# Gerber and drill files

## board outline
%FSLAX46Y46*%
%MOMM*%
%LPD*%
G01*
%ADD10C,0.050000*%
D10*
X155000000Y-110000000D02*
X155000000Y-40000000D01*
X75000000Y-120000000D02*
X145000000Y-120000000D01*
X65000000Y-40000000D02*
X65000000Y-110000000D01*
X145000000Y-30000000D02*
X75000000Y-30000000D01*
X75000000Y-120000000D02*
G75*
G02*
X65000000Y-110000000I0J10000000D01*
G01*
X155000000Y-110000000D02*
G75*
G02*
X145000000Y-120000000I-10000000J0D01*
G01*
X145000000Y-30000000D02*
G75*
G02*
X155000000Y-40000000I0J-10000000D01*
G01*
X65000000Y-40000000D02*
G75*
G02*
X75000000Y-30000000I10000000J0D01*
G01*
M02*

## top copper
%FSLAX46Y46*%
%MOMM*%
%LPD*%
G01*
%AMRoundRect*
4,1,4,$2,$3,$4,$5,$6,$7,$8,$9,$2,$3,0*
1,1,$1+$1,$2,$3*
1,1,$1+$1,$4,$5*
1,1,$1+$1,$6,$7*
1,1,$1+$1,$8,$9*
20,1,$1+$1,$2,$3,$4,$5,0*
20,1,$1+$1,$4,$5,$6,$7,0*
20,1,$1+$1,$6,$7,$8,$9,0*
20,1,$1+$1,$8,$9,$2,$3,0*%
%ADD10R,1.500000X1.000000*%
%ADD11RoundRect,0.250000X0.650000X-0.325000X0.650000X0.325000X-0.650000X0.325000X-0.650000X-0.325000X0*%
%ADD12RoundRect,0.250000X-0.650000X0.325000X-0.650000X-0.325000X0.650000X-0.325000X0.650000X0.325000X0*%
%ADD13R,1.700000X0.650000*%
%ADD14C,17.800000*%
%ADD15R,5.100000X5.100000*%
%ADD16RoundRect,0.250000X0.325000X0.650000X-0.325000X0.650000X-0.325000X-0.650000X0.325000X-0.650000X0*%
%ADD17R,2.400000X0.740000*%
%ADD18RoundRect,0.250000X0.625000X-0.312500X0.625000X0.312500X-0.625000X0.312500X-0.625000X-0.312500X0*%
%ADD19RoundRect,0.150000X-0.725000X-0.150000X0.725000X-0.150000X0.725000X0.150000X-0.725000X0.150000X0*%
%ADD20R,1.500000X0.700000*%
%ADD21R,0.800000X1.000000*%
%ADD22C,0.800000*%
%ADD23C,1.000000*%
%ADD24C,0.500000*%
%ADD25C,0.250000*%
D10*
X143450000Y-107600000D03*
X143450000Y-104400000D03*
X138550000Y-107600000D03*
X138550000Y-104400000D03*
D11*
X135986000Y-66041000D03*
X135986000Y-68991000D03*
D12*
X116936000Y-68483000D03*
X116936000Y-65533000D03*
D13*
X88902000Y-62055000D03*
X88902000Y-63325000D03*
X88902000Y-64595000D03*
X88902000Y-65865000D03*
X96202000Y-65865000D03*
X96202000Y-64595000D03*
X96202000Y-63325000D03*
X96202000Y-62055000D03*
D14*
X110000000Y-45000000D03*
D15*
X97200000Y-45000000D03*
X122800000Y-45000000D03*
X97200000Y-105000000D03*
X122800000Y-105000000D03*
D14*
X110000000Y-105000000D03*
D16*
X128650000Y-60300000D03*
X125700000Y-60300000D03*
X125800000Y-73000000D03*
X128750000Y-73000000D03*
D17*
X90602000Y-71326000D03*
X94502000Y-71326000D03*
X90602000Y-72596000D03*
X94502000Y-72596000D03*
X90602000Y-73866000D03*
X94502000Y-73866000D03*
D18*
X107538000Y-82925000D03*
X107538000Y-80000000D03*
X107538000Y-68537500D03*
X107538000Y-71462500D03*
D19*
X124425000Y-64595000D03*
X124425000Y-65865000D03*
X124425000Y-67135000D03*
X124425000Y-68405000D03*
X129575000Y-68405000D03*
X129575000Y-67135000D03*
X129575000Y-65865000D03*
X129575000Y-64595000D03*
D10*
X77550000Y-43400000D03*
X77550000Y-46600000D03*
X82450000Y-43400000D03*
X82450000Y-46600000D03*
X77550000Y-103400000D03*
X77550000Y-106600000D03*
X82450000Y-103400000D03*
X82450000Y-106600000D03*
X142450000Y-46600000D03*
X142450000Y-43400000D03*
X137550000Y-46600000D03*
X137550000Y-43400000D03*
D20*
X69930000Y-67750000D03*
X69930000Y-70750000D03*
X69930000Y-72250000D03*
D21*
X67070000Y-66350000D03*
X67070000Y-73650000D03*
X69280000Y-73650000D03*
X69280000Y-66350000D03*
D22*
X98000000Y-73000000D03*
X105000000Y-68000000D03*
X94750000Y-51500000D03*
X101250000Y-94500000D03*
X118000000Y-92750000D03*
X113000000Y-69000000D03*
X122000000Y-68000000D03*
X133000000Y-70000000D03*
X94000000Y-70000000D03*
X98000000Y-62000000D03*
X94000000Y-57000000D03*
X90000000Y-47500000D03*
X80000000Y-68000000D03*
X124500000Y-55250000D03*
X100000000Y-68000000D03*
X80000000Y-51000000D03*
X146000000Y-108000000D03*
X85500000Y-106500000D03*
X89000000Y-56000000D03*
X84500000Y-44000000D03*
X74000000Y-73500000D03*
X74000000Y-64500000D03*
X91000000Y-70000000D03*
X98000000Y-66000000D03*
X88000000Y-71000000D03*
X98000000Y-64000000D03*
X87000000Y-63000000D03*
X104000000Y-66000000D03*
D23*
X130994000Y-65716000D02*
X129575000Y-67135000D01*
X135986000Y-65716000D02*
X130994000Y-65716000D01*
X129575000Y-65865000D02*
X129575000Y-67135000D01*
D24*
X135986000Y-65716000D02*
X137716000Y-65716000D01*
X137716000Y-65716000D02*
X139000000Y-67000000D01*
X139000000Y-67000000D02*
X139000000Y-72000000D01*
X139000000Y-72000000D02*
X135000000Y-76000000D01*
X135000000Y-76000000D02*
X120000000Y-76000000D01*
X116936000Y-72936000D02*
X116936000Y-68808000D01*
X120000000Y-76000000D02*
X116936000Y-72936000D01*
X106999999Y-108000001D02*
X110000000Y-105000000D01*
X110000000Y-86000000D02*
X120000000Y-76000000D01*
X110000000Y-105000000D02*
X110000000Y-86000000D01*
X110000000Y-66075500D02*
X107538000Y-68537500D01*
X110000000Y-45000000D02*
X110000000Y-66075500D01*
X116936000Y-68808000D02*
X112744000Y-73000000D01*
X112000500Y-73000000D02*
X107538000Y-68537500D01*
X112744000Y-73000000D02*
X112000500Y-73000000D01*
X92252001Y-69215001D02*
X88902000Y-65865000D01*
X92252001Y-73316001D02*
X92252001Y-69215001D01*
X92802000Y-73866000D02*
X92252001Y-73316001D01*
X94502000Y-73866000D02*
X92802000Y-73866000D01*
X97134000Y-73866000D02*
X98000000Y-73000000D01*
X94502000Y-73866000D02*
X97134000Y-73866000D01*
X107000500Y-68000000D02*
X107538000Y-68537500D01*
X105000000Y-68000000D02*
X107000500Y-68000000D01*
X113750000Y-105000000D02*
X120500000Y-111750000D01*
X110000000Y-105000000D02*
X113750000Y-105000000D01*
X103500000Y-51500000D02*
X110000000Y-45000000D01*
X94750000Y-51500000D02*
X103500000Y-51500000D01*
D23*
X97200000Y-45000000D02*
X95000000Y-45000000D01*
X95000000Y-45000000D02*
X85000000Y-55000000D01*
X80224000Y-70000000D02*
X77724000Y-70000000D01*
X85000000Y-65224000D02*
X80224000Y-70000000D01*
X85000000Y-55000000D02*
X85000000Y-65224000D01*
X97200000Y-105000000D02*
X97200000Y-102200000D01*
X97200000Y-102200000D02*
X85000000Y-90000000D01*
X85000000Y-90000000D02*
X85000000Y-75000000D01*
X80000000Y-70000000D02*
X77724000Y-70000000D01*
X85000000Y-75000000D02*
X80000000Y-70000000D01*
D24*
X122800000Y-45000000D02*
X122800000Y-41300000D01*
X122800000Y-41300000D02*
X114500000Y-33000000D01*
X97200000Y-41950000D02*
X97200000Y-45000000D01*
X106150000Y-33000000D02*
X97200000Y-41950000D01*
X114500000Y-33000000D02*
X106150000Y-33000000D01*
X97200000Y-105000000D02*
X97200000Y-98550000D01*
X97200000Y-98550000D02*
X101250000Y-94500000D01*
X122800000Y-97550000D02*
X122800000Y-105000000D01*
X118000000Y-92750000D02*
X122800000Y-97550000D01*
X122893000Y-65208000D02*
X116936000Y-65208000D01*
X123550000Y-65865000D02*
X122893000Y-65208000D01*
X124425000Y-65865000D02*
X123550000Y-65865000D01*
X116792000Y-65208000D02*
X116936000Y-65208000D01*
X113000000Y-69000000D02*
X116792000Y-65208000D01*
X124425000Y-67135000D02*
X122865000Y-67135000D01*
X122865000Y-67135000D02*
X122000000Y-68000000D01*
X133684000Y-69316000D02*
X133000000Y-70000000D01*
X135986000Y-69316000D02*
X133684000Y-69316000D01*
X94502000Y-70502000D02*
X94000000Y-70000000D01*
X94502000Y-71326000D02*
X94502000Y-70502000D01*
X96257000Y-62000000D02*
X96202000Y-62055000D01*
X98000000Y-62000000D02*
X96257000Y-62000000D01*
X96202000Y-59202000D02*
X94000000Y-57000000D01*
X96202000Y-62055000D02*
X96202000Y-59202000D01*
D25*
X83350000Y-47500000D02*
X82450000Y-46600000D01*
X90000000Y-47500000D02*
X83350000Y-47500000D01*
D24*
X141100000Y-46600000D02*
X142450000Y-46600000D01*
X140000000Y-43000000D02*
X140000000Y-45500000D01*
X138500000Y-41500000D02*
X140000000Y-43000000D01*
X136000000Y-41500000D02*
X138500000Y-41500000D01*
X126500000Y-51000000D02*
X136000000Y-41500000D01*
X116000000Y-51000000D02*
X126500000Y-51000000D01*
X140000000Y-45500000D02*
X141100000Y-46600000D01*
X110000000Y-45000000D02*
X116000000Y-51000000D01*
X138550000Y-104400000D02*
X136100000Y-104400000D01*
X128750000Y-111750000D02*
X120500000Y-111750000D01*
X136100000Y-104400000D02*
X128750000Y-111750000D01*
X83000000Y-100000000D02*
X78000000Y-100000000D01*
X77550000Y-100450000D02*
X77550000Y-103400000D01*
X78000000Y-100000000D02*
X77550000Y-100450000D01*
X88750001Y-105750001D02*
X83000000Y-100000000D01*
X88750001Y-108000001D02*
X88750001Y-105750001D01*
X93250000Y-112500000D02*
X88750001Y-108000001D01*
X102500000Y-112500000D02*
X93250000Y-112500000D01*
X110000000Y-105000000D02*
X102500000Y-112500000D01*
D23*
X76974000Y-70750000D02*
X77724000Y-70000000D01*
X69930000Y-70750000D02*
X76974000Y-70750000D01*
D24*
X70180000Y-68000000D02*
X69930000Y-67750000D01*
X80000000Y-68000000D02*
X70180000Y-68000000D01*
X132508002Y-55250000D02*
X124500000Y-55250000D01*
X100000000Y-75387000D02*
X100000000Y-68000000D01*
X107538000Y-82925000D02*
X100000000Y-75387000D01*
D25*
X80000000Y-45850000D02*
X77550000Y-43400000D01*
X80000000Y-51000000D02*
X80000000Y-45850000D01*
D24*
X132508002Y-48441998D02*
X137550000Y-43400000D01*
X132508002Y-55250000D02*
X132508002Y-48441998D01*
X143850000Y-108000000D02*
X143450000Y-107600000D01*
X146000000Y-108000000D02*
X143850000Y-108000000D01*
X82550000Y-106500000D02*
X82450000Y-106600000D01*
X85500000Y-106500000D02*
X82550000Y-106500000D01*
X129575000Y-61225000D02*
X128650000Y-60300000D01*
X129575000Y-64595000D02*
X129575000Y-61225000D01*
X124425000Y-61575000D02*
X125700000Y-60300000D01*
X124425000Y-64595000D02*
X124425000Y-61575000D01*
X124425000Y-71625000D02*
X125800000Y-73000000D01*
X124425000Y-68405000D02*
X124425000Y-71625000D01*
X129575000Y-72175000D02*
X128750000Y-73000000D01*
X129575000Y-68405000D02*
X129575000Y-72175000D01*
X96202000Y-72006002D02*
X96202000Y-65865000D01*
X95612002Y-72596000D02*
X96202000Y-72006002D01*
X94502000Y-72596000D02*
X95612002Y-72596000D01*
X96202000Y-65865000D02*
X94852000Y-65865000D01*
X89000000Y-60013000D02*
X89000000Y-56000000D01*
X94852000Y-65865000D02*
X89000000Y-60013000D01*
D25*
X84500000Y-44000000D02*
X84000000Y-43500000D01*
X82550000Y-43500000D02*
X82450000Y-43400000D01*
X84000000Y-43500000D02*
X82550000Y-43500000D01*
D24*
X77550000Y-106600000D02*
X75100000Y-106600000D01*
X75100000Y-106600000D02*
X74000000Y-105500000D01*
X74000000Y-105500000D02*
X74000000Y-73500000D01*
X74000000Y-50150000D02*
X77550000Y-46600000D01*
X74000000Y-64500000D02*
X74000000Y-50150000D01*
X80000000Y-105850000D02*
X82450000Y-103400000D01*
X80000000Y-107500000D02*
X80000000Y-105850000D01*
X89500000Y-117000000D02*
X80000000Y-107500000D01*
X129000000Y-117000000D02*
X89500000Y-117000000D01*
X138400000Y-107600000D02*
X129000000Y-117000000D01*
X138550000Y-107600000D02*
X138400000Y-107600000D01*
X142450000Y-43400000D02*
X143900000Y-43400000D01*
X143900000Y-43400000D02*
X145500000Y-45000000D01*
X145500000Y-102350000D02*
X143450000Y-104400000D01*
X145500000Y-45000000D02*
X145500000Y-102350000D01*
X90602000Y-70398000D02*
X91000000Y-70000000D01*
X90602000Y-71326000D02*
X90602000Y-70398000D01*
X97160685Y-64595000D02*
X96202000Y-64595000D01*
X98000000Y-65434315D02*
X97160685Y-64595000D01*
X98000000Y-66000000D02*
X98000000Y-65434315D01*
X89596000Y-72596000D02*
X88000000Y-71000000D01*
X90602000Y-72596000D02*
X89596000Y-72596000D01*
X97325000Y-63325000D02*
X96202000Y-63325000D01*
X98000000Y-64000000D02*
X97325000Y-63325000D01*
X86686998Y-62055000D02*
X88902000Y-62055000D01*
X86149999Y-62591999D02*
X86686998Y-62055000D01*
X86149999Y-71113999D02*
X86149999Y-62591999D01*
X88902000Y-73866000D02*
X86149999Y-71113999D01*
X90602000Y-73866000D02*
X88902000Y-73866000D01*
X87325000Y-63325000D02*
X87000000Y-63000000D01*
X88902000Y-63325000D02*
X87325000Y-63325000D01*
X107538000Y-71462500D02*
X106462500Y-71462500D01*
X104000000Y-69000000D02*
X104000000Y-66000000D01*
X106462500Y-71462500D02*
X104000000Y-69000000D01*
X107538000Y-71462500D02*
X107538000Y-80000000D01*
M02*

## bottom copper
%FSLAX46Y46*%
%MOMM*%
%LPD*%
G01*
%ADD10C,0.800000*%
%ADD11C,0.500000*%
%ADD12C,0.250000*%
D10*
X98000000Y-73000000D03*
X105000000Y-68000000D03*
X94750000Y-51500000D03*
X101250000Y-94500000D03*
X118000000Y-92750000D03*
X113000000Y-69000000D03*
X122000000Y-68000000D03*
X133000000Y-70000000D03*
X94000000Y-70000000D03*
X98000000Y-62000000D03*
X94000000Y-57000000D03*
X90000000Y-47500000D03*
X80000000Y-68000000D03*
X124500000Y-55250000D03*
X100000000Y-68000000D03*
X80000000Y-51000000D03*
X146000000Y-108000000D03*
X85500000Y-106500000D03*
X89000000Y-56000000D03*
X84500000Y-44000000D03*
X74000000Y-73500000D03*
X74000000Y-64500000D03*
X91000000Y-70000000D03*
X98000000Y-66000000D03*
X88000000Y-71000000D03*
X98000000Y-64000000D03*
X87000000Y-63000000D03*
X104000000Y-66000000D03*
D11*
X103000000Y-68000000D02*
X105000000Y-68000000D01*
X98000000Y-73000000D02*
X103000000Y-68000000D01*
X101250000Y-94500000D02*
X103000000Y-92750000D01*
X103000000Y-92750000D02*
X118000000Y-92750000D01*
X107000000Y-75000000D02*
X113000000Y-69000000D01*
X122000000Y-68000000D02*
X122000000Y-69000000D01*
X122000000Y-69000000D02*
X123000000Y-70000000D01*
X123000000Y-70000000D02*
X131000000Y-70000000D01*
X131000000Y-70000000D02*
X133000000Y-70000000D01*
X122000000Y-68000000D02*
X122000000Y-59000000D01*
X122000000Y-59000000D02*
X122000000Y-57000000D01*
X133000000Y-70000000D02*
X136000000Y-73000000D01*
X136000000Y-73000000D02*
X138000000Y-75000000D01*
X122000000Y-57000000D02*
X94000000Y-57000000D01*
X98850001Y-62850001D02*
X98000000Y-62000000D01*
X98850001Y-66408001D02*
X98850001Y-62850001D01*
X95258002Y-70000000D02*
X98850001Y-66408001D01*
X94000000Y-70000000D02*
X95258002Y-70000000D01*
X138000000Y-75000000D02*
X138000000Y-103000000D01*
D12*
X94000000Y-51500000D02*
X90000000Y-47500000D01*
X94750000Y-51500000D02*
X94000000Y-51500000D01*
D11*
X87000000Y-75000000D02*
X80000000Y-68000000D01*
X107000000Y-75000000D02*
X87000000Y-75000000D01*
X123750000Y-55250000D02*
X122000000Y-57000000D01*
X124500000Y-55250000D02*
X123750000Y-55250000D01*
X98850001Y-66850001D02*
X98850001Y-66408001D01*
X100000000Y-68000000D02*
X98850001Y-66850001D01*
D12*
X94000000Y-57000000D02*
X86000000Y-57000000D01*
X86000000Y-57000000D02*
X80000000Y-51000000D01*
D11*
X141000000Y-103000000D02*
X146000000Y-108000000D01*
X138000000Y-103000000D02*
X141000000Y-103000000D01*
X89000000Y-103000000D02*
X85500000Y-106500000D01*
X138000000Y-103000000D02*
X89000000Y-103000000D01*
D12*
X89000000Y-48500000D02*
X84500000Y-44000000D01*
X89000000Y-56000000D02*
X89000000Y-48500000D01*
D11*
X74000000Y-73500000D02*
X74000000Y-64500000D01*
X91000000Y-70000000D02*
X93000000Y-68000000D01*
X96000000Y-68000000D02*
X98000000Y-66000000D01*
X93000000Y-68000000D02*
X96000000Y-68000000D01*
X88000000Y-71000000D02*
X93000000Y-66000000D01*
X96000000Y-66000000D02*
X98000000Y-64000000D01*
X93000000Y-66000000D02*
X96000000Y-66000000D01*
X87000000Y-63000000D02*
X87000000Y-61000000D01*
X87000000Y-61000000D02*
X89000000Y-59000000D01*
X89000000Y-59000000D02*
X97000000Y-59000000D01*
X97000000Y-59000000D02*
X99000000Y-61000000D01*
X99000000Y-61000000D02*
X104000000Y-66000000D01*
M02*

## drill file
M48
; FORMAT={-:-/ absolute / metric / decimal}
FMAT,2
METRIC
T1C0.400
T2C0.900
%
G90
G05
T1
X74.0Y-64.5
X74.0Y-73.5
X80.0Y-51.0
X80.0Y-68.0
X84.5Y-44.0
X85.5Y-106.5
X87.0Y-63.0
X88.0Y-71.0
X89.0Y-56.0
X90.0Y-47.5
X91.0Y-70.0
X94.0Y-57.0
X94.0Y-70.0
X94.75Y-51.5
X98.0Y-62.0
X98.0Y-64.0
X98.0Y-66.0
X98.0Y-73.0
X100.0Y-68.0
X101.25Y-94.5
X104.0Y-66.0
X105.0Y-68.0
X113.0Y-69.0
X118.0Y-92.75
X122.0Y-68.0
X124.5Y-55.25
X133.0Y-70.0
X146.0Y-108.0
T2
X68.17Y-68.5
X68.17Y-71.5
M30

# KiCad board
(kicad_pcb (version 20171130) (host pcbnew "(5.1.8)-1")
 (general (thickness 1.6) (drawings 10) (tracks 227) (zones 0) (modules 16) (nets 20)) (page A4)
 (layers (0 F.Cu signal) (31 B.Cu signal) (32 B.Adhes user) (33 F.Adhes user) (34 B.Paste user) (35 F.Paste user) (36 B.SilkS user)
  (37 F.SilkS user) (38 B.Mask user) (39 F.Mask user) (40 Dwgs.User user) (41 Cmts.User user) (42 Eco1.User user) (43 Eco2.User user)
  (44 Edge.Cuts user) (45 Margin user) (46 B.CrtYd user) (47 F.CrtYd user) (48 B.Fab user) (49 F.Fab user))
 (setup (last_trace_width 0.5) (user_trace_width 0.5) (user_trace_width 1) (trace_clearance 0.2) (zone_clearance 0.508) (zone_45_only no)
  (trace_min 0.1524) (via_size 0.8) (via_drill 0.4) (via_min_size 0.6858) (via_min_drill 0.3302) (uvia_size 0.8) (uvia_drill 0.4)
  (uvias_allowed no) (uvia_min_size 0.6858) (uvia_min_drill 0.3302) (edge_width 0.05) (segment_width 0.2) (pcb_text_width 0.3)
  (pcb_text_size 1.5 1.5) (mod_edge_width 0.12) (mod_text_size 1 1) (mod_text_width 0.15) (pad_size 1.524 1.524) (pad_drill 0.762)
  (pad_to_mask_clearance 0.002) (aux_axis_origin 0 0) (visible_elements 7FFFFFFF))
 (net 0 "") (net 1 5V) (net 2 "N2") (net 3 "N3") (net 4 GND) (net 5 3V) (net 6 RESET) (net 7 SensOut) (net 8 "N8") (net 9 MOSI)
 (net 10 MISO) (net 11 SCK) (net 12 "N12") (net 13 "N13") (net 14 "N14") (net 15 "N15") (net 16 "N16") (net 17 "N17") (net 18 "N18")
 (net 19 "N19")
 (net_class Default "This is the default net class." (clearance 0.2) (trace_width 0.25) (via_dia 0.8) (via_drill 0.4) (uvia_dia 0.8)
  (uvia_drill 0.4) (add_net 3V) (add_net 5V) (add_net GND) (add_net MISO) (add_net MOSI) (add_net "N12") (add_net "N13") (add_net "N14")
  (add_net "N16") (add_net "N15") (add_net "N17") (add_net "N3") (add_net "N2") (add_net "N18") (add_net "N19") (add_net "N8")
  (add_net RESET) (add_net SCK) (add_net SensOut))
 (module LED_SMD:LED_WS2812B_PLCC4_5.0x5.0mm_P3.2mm (layer F.Cu) (at 141 106 180)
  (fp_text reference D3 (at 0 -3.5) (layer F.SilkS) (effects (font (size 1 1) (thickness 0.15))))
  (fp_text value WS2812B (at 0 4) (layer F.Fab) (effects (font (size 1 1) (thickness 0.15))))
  (pad 1 smd rect (at -2.45 -1.6 180) (size 1.5 1) (layers F.Cu F.Paste F.Mask) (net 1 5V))
  (pad 2 smd rect (at -2.45 1.6 180) (size 1.5 1) (layers F.Cu F.Paste F.Mask) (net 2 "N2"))
  (pad 4 smd rect (at 2.45 -1.6 180) (size 1.5 1) (layers F.Cu F.Paste F.Mask) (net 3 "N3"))
  (pad 3 smd rect (at 2.45 1.6 180) (size 1.5 1) (layers F.Cu F.Paste F.Mask) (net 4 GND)))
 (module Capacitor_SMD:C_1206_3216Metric (layer F.Cu) (at 135.986 67.516 90)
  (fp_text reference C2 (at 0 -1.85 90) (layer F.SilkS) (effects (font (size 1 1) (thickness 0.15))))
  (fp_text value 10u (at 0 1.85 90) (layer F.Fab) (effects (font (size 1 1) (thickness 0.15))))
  (pad 2 smd roundrect (at 1.475 0 90) (size 1.15 1.8) (layers F.Cu F.Paste F.Mask) (roundrect_rratio 0.217391) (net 4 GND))
  (pad 1 smd roundrect (at -1.475 0 90) (size 1.15 1.8) (layers F.Cu F.Paste F.Mask) (roundrect_rratio 0.217391) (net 1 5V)))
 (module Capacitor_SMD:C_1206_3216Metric (layer F.Cu) (at 116.936 67.008 270)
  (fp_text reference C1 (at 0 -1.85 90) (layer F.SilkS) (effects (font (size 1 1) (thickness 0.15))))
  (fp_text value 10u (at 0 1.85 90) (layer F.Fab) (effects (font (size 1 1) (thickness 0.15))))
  (pad 2 smd roundrect (at 1.475 0 270) (size 1.15 1.8) (layers F.Cu F.Paste F.Mask) (roundrect_rratio 0.217391) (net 4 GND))
  (pad 1 smd roundrect (at -1.475 0 270) (size 1.15 1.8) (layers F.Cu F.Paste F.Mask) (roundrect_rratio 0.217391) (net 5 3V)))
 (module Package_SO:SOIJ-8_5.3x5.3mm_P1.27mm (layer F.Cu) (at 92.552 63.96)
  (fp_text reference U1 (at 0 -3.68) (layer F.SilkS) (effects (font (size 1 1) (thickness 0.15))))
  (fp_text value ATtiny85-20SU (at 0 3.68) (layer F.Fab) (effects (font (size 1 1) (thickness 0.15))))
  (pad 1 smd rect (at -3.65 -1.905) (size 1.7 0.65) (layers F.Cu F.Paste F.Mask) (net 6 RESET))
  (pad 2 smd rect (at -3.65 -0.635) (size 1.7 0.65) (layers F.Cu F.Paste F.Mask) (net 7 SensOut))
  (pad 3 smd rect (at -3.65 0.635) (size 1.7 0.65) (layers F.Cu F.Paste F.Mask) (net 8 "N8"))
  (pad 4 smd rect (at -3.65 1.905) (size 1.7 0.65) (layers F.Cu F.Paste F.Mask) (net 4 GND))
  (pad 5 smd rect (at 3.65 1.905) (size 1.7 0.65) (layers F.Cu F.Paste F.Mask) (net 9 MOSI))
  (pad 6 smd rect (at 3.65 0.635) (size 1.7 0.65) (layers F.Cu F.Paste F.Mask) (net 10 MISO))
  (pad 7 smd rect (at 3.65 -0.635) (size 1.7 0.65) (layers F.Cu F.Paste F.Mask) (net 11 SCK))
  (pad 8 smd rect (at 3.65 -1.905) (size 1.7 0.65) (layers F.Cu F.Paste F.Mask) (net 1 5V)))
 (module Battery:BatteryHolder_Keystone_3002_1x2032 (layer F.Cu) (at 110 45)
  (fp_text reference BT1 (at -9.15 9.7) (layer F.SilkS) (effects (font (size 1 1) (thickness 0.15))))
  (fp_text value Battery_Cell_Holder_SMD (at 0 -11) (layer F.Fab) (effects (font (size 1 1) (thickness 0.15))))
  (pad 2 smd circle (at 0 0) (size 17.8 17.8) (layers F.Cu F.Mask) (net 4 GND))
  (pad 1 smd rect (at -12.8 0) (size 5.1 5.1) (layers F.Cu F.Paste F.Mask) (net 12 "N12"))
  (pad 1 smd rect (at 12.8 0) (size 5.1 5.1) (layers F.Cu F.Paste F.Mask) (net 12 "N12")))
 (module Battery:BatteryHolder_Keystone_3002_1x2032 (layer F.Cu) (at 110 105 180)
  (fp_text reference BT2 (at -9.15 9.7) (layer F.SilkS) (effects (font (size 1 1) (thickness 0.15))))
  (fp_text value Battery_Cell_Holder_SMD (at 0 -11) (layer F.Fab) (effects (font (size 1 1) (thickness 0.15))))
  (pad 1 smd rect (at 12.8 0 180) (size 5.1 5.1) (layers F.Cu F.Paste F.Mask) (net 12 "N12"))
  (pad 1 smd rect (at -12.8 0 180) (size 5.1 5.1) (layers F.Cu F.Paste F.Mask) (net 12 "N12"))
  (pad 2 smd circle (at 0 0 180) (size 17.8 17.8) (layers F.Cu F.Mask) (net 4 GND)))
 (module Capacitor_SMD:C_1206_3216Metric (layer F.Cu) (at 127.175 60.3 180)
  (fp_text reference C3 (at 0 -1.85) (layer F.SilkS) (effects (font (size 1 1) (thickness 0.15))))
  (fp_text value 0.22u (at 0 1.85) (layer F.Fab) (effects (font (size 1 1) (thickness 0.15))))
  (pad 1 smd roundrect (at -1.475 0 180) (size 1.15 1.8) (layers F.Cu F.Paste F.Mask) (roundrect_rratio 0.217391) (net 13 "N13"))
  (pad 2 smd roundrect (at 1.475 0 180) (size 1.15 1.8) (layers F.Cu F.Paste F.Mask) (roundrect_rratio 0.217391) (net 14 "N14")))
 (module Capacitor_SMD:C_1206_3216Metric (layer F.Cu) (at 127.275 73 180)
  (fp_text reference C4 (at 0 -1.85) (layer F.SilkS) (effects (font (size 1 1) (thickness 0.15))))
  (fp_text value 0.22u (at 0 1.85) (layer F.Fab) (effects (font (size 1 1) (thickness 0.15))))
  (pad 2 smd roundrect (at 1.475 0 180) (size 1.15 1.8) (layers F.Cu F.Paste F.Mask) (roundrect_rratio 0.217391) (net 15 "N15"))
  (pad 1 smd roundrect (at -1.475 0 180) (size 1.15 1.8) (layers F.Cu F.Paste F.Mask) (roundrect_rratio 0.217391) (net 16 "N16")))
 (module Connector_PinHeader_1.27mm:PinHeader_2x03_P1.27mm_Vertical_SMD (layer F.Cu) (at 92.552 72.596)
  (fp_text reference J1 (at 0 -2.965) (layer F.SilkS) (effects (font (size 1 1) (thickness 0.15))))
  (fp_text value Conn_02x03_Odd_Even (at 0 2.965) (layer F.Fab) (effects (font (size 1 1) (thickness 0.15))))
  (pad 1 smd rect (at -1.95 -1.27) (size 2.4 0.74) (layers F.Cu F.Paste F.Mask) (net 10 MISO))
  (pad 2 smd rect (at 1.95 -1.27) (size 2.4 0.74) (layers F.Cu F.Paste F.Mask) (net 1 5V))
  (pad 3 smd rect (at -1.95 0) (size 2.4 0.74) (layers F.Cu F.Paste F.Mask) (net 11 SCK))
  (pad 4 smd rect (at 1.95 0) (size 2.4 0.74) (layers F.Cu F.Paste F.Mask) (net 9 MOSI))
  (pad 5 smd rect (at -1.95 1.27) (size 2.4 0.74) (layers F.Cu F.Paste F.Mask) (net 6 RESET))
  (pad 6 smd rect (at 1.95 1.27) (size 2.4 0.74) (layers F.Cu F.Paste F.Mask) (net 4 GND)))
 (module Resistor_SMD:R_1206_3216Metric (layer F.Cu) (at 107.538 81.4625 90)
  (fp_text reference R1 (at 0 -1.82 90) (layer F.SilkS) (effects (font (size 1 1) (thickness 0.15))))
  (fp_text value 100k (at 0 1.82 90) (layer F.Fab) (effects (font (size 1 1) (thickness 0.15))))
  (pad 1 smd roundrect (at -1.4625 0 90) (size 1.125 1.75) (layers F.Cu F.Paste F.Mask) (roundrect_rratio 0.222222) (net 1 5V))
  (pad 2 smd roundrect (at 1.4625 0 90) (size 1.125 1.75) (layers F.Cu F.Paste F.Mask) (roundrect_rratio 0.222222) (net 7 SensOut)))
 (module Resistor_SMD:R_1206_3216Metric (layer F.Cu) (at 107.538 70 90)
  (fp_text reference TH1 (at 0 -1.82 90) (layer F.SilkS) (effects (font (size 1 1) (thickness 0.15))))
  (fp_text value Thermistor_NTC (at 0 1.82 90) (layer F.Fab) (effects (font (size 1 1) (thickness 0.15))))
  (pad 2 smd roundrect (at 1.4625 0 90) (size 1.125 1.75) (layers F.Cu F.Paste F.Mask) (roundrect_rratio 0.222222) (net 4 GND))
  (pad 1 smd roundrect (at -1.4625 0 90) (size 1.125 1.75) (layers F.Cu F.Paste F.Mask) (roundrect_rratio 0.222222) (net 7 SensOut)))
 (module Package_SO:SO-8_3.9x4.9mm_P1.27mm (layer F.Cu) (at 127 66.5)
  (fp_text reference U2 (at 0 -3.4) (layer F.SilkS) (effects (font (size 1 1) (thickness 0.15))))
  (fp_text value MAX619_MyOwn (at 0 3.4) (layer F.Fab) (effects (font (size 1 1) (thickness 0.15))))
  (pad 1 smd roundrect (at -2.575 -1.905) (size 1.75 0.6) (layers F.Cu F.Paste F.Mask) (roundrect_rratio 0.25) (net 14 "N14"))
  (pad 2 smd roundrect (at -2.575 -0.635) (size 1.75 0.6) (layers F.Cu F.Paste F.Mask) (roundrect_rratio 0.25) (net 5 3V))
  (pad 3 smd roundrect (at -2.575 0.635) (size 1.75 0.6) (layers F.Cu F.Paste F.Mask) (roundrect_rratio 0.25) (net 1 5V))
  (pad 4 smd roundrect (at -2.575 1.905) (size 1.75 0.6) (layers F.Cu F.Paste F.Mask) (roundrect_rratio 0.25) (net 15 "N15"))
  (pad 5 smd roundrect (at 2.575 1.905) (size 1.75 0.6) (layers F.Cu F.Paste F.Mask) (roundrect_rratio 0.25) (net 16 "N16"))
  (pad 6 smd roundrect (at 2.575 0.635) (size 1.75 0.6) (layers F.Cu F.Paste F.Mask) (roundrect_rratio 0.25) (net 4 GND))
  (pad 7 smd roundrect (at 2.575 -0.635) (size 1.75 0.6) (layers F.Cu F.Paste F.Mask) (roundrect_rratio 0.25) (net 4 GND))
  (pad 8 smd roundrect (at 2.575 -1.905) (size 1.75 0.6) (layers F.Cu F.Paste F.Mask) (roundrect_rratio 0.25) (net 13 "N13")))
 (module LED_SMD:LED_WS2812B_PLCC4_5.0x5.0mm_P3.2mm (layer F.Cu) (at 80 45)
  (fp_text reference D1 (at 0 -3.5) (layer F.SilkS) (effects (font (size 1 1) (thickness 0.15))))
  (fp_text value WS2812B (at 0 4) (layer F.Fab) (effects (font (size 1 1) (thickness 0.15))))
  (pad 1 smd rect (at -2.45 -1.6) (size 1.5 1) (layers F.Cu F.Paste F.Mask) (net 1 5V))
  (pad 2 smd rect (at -2.45 1.6) (size 1.5 1) (layers F.Cu F.Paste F.Mask) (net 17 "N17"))
  (pad 4 smd rect (at 2.45 -1.6) (size 1.5 1) (layers F.Cu F.Paste F.Mask) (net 9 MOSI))
  (pad 3 smd rect (at 2.45 1.6) (size 1.5 1) (layers F.Cu F.Paste F.Mask) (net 4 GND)))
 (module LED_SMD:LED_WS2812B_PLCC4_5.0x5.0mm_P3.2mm (layer F.Cu) (at 80 105 180)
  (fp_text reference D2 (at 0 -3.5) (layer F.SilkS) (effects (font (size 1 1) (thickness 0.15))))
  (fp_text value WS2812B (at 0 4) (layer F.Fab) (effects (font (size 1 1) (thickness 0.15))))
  (pad 3 smd rect (at 2.45 1.6 180) (size 1.5 1) (layers F.Cu F.Paste F.Mask) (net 4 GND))
  (pad 4 smd rect (at 2.45 -1.6 180) (size 1.5 1) (layers F.Cu F.Paste F.Mask) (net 17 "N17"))
  (pad 2 smd rect (at -2.45 1.6 180) (size 1.5 1) (layers F.Cu F.Paste F.Mask) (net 3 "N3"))
  (pad 1 smd rect (at -2.45 -1.6 180) (size 1.5 1) (layers F.Cu F.Paste F.Mask) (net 1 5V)))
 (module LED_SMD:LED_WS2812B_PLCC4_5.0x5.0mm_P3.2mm (layer F.Cu) (at 140 45)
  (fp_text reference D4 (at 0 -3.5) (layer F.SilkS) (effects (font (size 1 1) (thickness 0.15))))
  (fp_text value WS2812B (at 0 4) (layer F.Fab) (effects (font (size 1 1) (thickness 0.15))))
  (pad 3 smd rect (at 2.45 1.6) (size 1.5 1) (layers F.Cu F.Paste F.Mask) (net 4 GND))
  (pad 4 smd rect (at 2.45 -1.6) (size 1.5 1) (layers F.Cu F.Paste F.Mask) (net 2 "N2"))
  (pad 2 smd rect (at -2.45 1.6) (size 1.5 1) (layers F.Cu F.Paste F.Mask) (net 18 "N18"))
  (pad 1 smd rect (at -2.45 -1.6) (size 1.5 1) (layers F.Cu F.Paste F.Mask) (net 1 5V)))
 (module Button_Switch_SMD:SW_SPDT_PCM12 (layer F.Cu) (at 68.5 70 270)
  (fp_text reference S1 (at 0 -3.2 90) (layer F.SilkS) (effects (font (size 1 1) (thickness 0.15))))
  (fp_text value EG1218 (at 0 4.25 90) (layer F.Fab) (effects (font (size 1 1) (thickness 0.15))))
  (pad "" np_thru_hole circle (at -1.5 0.33 270) (size 0.9 0.9) (drill 0.9) (layers *.Cu *.Mask))
  (pad "" np_thru_hole circle (at 1.5 0.33 270) (size 0.9 0.9) (drill 0.9) (layers *.Cu *.Mask))
  (pad 1 smd rect (at -2.25 -1.43 270) (size 0.7 1.5) (layers F.Cu F.Paste F.Mask) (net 5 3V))
  (pad 2 smd rect (at 0.75 -1.43 270) (size 0.7 1.5) (layers F.Cu F.Paste F.Mask) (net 12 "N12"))
  (pad 3 smd rect (at 2.25 -1.43 270) (size 0.7 1.5) (layers F.Cu F.Paste F.Mask) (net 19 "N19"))
  (pad "" smd rect (at -3.65 1.43 270) (size 1 0.8) (layers F.Cu F.Paste F.Mask))
  (pad "" smd rect (at 3.65 1.43 270) (size 1 0.8) (layers F.Cu F.Paste F.Mask))
  (pad "" smd rect (at 3.65 -0.78 270) (size 1 0.8) (layers F.Cu F.Paste F.Mask))
  (pad "" smd rect (at -3.65 -0.78 270) (size 1 0.8) (layers F.Cu F.Paste F.Mask)))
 (gr_line (start 155 110) (end 155 40) (layer Edge.Cuts) (width 0.05))
 (gr_line (start 75 120) (end 145 120) (layer Edge.Cuts) (width 0.05))
 (gr_line (start 65 40) (end 65 110) (layer Edge.Cuts) (width 0.05))
 (gr_line (start 145 30) (end 75 30) (layer Edge.Cuts) (width 0.05))
 (gr_arc (start 75 110) (end 65 110) (angle -90) (layer Edge.Cuts) (width 0.05))
 (gr_arc (start 145 110) (end 145 120) (angle -90) (layer Edge.Cuts) (width 0.05))
 (gr_arc (start 145 40) (end 155 40) (angle -90) (layer Edge.Cuts) (width 0.05))
 (gr_arc (start 75 40) (end 75 30) (angle -90) (layer Edge.Cuts) (width 0.05))
 (segment (start 130.994 65.716) (end 129.575 67.135) (width 1) (layer F.Cu) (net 4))
 (segment (start 135.986 65.716) (end 130.994 65.716) (width 1) (layer F.Cu) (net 4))
 (segment (start 129.575 65.865) (end 129.575 67.135) (width 1) (layer F.Cu) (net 4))
 (segment (start 135.986 65.716) (end 137.716 65.716) (width 0.5) (layer F.Cu) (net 4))
 (segment (start 137.716 65.716) (end 139 67) (width 0.5) (layer F.Cu) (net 4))
 (segment (start 139 67) (end 139 72) (width 0.5) (layer F.Cu) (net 4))
 (segment (start 139 72) (end 135 76) (width 0.5) (layer F.Cu) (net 4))
 (segment (start 135 76) (end 120 76) (width 0.5) (layer F.Cu) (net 4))
 (segment (start 116.936 72.936) (end 116.936 68.808) (width 0.5) (layer F.Cu) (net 4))
 (segment (start 120 76) (end 116.936 72.936) (width 0.5) (layer F.Cu) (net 4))
 (segment (start 106.999999 108.000001) (end 110 105) (width 0.5) (layer F.Cu) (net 4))
 (segment (start 110 86) (end 120 76) (width 0.5) (layer F.Cu) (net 4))
 (segment (start 110 105) (end 110 86) (width 0.5) (layer F.Cu) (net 4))
 (segment (start 110 66.0755) (end 107.538 68.5375) (width 0.5) (layer F.Cu) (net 4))
 (segment (start 110 45) (end 110 66.0755) (width 0.5) (layer F.Cu) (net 4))
 (segment (start 116.936 68.808) (end 112.744 73) (width 0.5) (layer F.Cu) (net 4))
 (segment (start 112.0005 73) (end 107.538 68.5375) (width 0.5) (layer F.Cu) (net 4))
 (segment (start 112.744 73) (end 112.0005 73) (width 0.5) (layer F.Cu) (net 4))
 (segment (start 92.252001 69.215001) (end 88.902 65.865) (width 0.5) (layer F.Cu) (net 4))
 (segment (start 92.252001 73.316001) (end 92.252001 69.215001) (width 0.5) (layer F.Cu) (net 4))
 (segment (start 92.802 73.866) (end 92.252001 73.316001) (width 0.5) (layer F.Cu) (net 4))
 (segment (start 94.502 73.866) (end 92.802 73.866) (width 0.5) (layer F.Cu) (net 4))
 (via (at 98 73) (size 0.8) (drill 0.4) (layers F.Cu B.Cu) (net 4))
 (segment (start 97.134 73.866) (end 98 73) (width 0.5) (layer F.Cu) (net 4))
 (segment (start 94.502 73.866) (end 97.134 73.866) (width 0.5) (layer F.Cu) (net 4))
 (via (at 105 68) (size 0.8) (drill 0.4) (layers F.Cu B.Cu) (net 4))
 (segment (start 103 68) (end 105 68) (width 0.5) (layer B.Cu) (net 4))
 (segment (start 98 73) (end 103 68) (width 0.5) (layer B.Cu) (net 4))
 (segment (start 107.0005 68) (end 107.538 68.5375) (width 0.5) (layer F.Cu) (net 4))
 (segment (start 105 68) (end 107.0005 68) (width 0.5) (layer F.Cu) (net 4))
 (segment (start 113.75 105) (end 120.5 111.75) (width 0.5) (layer F.Cu) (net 4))
 (segment (start 110 105) (end 113.75 105) (width 0.5) (layer F.Cu) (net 4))
 (via (at 94.75 51.5) (size 0.8) (drill 0.4) (layers F.Cu B.Cu) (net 4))
 (segment (start 103.5 51.5) (end 110 45) (width 0.5) (layer F.Cu) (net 4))
 (segment (start 94.75 51.5) (end 103.5 51.5) (width 0.5) (layer F.Cu) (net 4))
 (segment (start 97.2 45) (end 95 45) (width 1) (layer F.Cu) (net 12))
 (segment (start 95 45) (end 85 55) (width 1) (layer F.Cu) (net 12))
 (segment (start 80.224 70) (end 77.724 70) (width 1) (layer F.Cu) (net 12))
 (segment (start 85 65.224) (end 80.224 70) (width 1) (layer F.Cu) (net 12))
 (segment (start 85 55) (end 85 65.224) (width 1) (layer F.Cu) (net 12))
 (segment (start 97.2 105) (end 97.2 102.2) (width 1) (layer F.Cu) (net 12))
 (segment (start 97.2 102.2) (end 85 90) (width 1) (layer F.Cu) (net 12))
 (segment (start 85 90) (end 85 75) (width 1) (layer F.Cu) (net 12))
 (segment (start 80 70) (end 77.724 70) (width 1) (layer F.Cu) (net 12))
 (segment (start 85 75) (end 80 70) (width 1) (layer F.Cu) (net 12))
 (segment (start 122.8 45) (end 122.8 41.3) (width 0.5) (layer F.Cu) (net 12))
 (segment (start 122.8 41.3) (end 114.5 33) (width 0.5) (layer F.Cu) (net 12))
 (segment (start 97.2 41.95) (end 97.2 45) (width 0.5) (layer F.Cu) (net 12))
 (segment (start 106.15 33) (end 97.2 41.95) (width 0.5) (layer F.Cu) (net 12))
 (segment (start 114.5 33) (end 106.15 33) (width 0.5) (layer F.Cu) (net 12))
 (segment (start 97.2 105) (end 97.2 98.55) (width 0.5) (layer F.Cu) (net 12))
 (via (at 101.25 94.5) (size 0.8) (drill 0.4) (layers F.Cu B.Cu) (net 12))
 (segment (start 97.2 98.55) (end 101.25 94.5) (width 0.5) (layer F.Cu) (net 12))
 (segment (start 101.25 94.5) (end 103 92.75) (width 0.5) (layer B.Cu) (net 12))
 (via (at 118 92.75) (size 0.8) (drill 0.4) (layers F.Cu B.Cu) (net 12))
 (segment (start 103 92.75) (end 118 92.75) (width 0.5) (layer B.Cu) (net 12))
 (segment (start 122.8 97.55) (end 122.8 105) (width 0.5) (layer F.Cu) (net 12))
 (segment (start 118 92.75) (end 122.8 97.55) (width 0.5) (layer F.Cu) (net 12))
 (segment (start 122.893 65.208) (end 116.936 65.208) (width 0.5) (layer F.Cu) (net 5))
 (segment (start 123.55 65.865) (end 122.893 65.208) (width 0.5) (layer F.Cu) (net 5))
 (segment (start 124.425 65.865) (end 123.55 65.865) (width 0.5) (layer F.Cu) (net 5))
 (via (at 113 69) (size 0.8) (drill 0.4) (layers F.Cu B.Cu) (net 5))
 (segment (start 107 75) (end 113 69) (width 0.5) (layer B.Cu) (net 5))
 (segment (start 116.792 65.208) (end 116.936 65.208) (width 0.5) (layer F.Cu) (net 5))
 (segment (start 113 69) (end 116.792 65.208) (width 0.5) (layer F.Cu) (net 5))
 (segment (start 124.425 67.135) (end 122.865 67.135) (width 0.5) (layer F.Cu) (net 1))
 (via (at 122 68) (size 0.8) (drill 0.4) (layers F.Cu B.Cu) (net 1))
 (segment (start 122.865 67.135) (end 122 68) (width 0.5) (layer F.Cu) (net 1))
 (segment (start 122 68) (end 122 69) (width 0.5) (layer B.Cu) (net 1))
 (segment (start 122 69) (end 123 70) (width 0.5) (layer B.Cu) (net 1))
 (segment (start 123 70) (end 131 70) (width 0.5) (layer B.Cu) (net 1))
 (segment (start 131 70) (end 133 70) (width 0.5) (layer B.Cu) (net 1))
 (via (at 133 70) (size 0.8) (drill 0.4) (layers F.Cu B.Cu) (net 1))
 (segment (start 133.684 69.316) (end 133 70) (width 0.5) (layer F.Cu) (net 1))
 (segment (start 135.986 69.316) (end 133.684 69.316) (width 0.5) (layer F.Cu) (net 1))
 (segment (start 122 68) (end 122 59) (width 0.5) (layer B.Cu) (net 1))
 (segment (start 122 59) (end 122 57) (width 0.5) (layer B.Cu) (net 1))
 (segment (start 133 70) (end 136 73) (width 0.5) (layer B.Cu) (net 1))
 (segment (start 136 73) (end 138 75) (width 0.5) (layer B.Cu) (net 1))
 (segment (start 122 57) (end 94 57) (width 0.5) (layer B.Cu) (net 1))
 (via (at 94 70) (size 0.8) (drill 0.4) (layers F.Cu B.Cu) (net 1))
 (segment (start 94.502 70.502) (end 94 70) (width 0.5) (layer F.Cu) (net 1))
 (segment (start 94.502 71.326) (end 94.502 70.502) (width 0.5) (layer F.Cu) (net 1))
 (via (at 98 62) (size 0.8) (drill 0.4) (layers F.Cu B.Cu) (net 1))
 (segment (start 98.850001 62.850001) (end 98 62) (width 0.5) (layer B.Cu) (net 1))
 (segment (start 98.850001 66.408001) (end 98.850001 62.850001) (width 0.5) (layer B.Cu) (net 1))
 (segment (start 95.258002 70) (end 98.850001 66.408001) (width 0.5) (layer B.Cu) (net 1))
 (segment (start 94 70) (end 95.258002 70) (width 0.5) (layer B.Cu) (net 1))
 (segment (start 96.257 62) (end 96.202 62.055) (width 0.5) (layer F.Cu) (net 1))
 (segment (start 98 62) (end 96.257 62) (width 0.5) (layer F.Cu) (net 1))
 (via (at 94 57) (size 0.8) (drill 0.4) (layers F.Cu B.Cu) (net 1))
 (segment (start 96.202 59.202) (end 94 57) (width 0.5) (layer F.Cu) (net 1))
 (segment (start 96.202 62.055) (end 96.202 59.202) (width 0.5) (layer F.Cu) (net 1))
 (segment (start 138 75) (end 138 103) (width 0.5) (layer B.Cu) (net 1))
 (via (at 90 47.5) (size 0.8) (drill 0.4) (layers F.Cu B.Cu) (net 4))
 (segment (start 94 51.5) (end 90 47.5) (width 0.25) (layer B.Cu) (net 4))
 (segment (start 94.75 51.5) (end 94 51.5) (width 0.25) (layer B.Cu) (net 4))
 (segment (start 83.35 47.5) (end 82.45 46.6) (width 0.25) (layer F.Cu) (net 4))
 (segment (start 90 47.5) (end 83.35 47.5) (width 0.25) (layer F.Cu) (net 4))
 (segment (start 141.1 46.6) (end 142.45 46.6) (width 0.5) (layer F.Cu) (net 4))
 (segment (start 140 43) (end 140 45.5) (width 0.5) (layer F.Cu) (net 4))
 (segment (start 138.5 41.5) (end 140 43) (width 0.5) (layer F.Cu) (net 4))
 (segment (start 136 41.5) (end 138.5 41.5) (width 0.5) (layer F.Cu) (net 4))
 (segment (start 126.5 51) (end 136 41.5) (width 0.5) (layer F.Cu) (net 4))
 (segment (start 116 51) (end 126.5 51) (width 0.5) (layer F.Cu) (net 4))
 (segment (start 140 45.5) (end 141.1 46.6) (width 0.5) (layer F.Cu) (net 4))
 (segment (start 110 45) (end 116 51) (width 0.5) (layer F.Cu) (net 4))
 (segment (start 138.55 104.4) (end 136.1 104.4) (width 0.5) (layer F.Cu) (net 4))
 (segment (start 128.75 111.75) (end 120.5 111.75) (width 0.5) (layer F.Cu) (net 4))
 (segment (start 136.1 104.4) (end 128.75 111.75) (width 0.5) (layer F.Cu) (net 4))
 (segment (start 83 100) (end 78 100) (width 0.5) (layer F.Cu) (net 4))
 (segment (start 77.55 100.45) (end 77.55 103.4) (width 0.5) (layer F.Cu) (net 4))
 (segment (start 78 100) (end 77.55 100.45) (width 0.5) (layer F.Cu) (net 4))
 (segment (start 88.750001 105.750001) (end 83 100) (width 0.5) (layer F.Cu) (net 4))
 (segment (start 88.750001 108.000001) (end 88.750001 105.750001) (width 0.5) (layer F.Cu) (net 4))
 (segment (start 93.25 112.5) (end 88.750001 108.000001) (width 0.5) (layer F.Cu) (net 4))
 (segment (start 102.5 112.5) (end 93.25 112.5) (width 0.5) (layer F.Cu) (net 4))
 (segment (start 110 105) (end 102.5 112.5) (width 0.5) (layer F.Cu) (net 4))
 (segment (start 76.974 70.75) (end 77.724 70) (width 1) (layer F.Cu) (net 12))
 (segment (start 69.93 70.75) (end 76.974 70.75) (width 1) (layer F.Cu) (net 12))
 (via (at 80 68) (size 0.8) (drill 0.4) (layers F.Cu B.Cu) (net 5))
 (segment (start 87 75) (end 80 68) (width 0.5) (layer B.Cu) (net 5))
 (segment (start 107 75) (end 87 75) (width 0.5) (layer B.Cu) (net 5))
 (segment (start 70.18 68) (end 69.93 67.75) (width 0.5) (layer F.Cu) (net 5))
 (segment (start 80 68) (end 70.18 68) (width 0.5) (layer F.Cu) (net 5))
 (via (at 124.5 55.25) (size 0.8) (drill 0.4) (layers F.Cu B.Cu) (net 1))
 (segment (start 132.508002 55.25) (end 124.5 55.25) (width 0.5) (layer F.Cu) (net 1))
 (segment (start 123.75 55.25) (end 122 57) (width 0.5) (layer B.Cu) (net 1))
 (segment (start 124.5 55.25) (end 123.75 55.25) (width 0.5) (layer B.Cu) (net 1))
 (via (at 100 68) (size 0.8) (drill 0.4) (layers F.Cu B.Cu) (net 1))
 (segment (start 100 75.387) (end 100 68) (width 0.5) (layer F.Cu) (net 1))
 (segment (start 107.538 82.925) (end 100 75.387) (width 0.5) (layer F.Cu) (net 1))
 (segment (start 98.850001 66.850001) (end 98.850001 66.408001) (width 0.5) (layer B.Cu) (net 1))
 (segment (start 100 68) (end 98.850001 66.850001) (width 0.5) (layer B.Cu) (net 1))
 (segment (start 94 57) (end 86 57) (width 0.25) (layer B.Cu) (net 1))
 (via (at 80 51) (size 0.8) (drill 0.4) (layers F.Cu B.Cu) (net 1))
 (segment (start 86 57) (end 80 51) (width 0.25) (layer B.Cu) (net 1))
 (segment (start 80 45.85) (end 77.55 43.4) (width 0.25) (layer F.Cu) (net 1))
 (segment (start 80 51) (end 80 45.85) (width 0.25) (layer F.Cu) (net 1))
 (segment (start 132.508002 48.441998) (end 137.55 43.4) (width 0.5) (layer F.Cu) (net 1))
 (segment (start 132.508002 55.25) (end 132.508002 48.441998) (width 0.5) (layer F.Cu) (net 1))
 (via (at 146 108) (size 0.8) (drill 0.4) (layers F.Cu B.Cu) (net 1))
 (segment (start 141 103) (end 146 108) (width 0.5) (layer B.Cu) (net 1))
 (segment (start 138 103) (end 141 103) (width 0.5) (layer B.Cu) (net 1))
 (segment (start 143.85 108) (end 143.45 107.6) (width 0.5) (layer F.Cu) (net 1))
 (segment (start 146 108) (end 143.85 108) (width 0.5) (layer F.Cu) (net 1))
 (via (at 85.5 106.5) (size 0.8) (drill 0.4) (layers F.Cu B.Cu) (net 1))
 (segment (start 89 103) (end 85.5 106.5) (width 0.5) (layer B.Cu) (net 1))
 (segment (start 138 103) (end 89 103) (width 0.5) (layer B.Cu) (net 1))
 (segment (start 82.55 106.5) (end 82.45 106.6) (width 0.5) (layer F.Cu) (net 1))
 (segment (start 85.5 106.5) (end 82.55 106.5) (width 0.5) (layer F.Cu) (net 1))
 (segment (start 129.575 61.225) (end 128.65 60.3) (width 0.5) (layer F.Cu) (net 13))
 (segment (start 129.575 64.595) (end 129.575 61.225) (width 0.5) (layer F.Cu) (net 13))
 (segment (start 124.425 61.575) (end 125.7 60.3) (width 0.5) (layer F.Cu) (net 14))
 (segment (start 124.425 64.595) (end 124.425 61.575) (width 0.5) (layer F.Cu) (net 14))
 (segment (start 124.425 71.625) (end 125.8 73) (width 0.5) (layer F.Cu) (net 15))
 (segment (start 124.425 68.405) (end 124.425 71.625) (width 0.5) (layer F.Cu) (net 15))
 (segment (start 129.575 72.175) (end 128.75 73) (width 0.5) (layer F.Cu) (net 16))
 (segment (start 129.575 68.405) (end 129.575 72.175) (width 0.5) (layer F.Cu) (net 16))
 (segment (start 96.202 72.006002) (end 96.202 65.865) (width 0.5) (layer F.Cu) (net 9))
 (segment (start 95.612002 72.596) (end 96.202 72.006002) (width 0.5) (layer F.Cu) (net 9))
 (segment (start 94.502 72.596) (end 95.612002 72.596) (width 0.5) (layer F.Cu) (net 9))
 (via (at 89 56) (size 0.8) (drill 0.4) (layers F.Cu B.Cu) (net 9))
 (segment (start 96.202 65.865) (end 94.852 65.865) (width 0.5) (layer F.Cu) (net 9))
 (segment (start 89 60.013) (end 89 56) (width 0.5) (layer F.Cu) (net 9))
 (segment (start 94.852 65.865) (end 89 60.013) (width 0.5) (layer F.Cu) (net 9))
 (via (at 84.5 44) (size 0.8) (drill 0.4) (layers F.Cu B.Cu) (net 9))
 (segment (start 89 48.5) (end 84.5 44) (width 0.25) (layer B.Cu) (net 9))
 (segment (start 89 56) (end 89 48.5) (width 0.25) (layer B.Cu) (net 9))
 (segment (start 84.5 44) (end 84 43.5) (width 0.25) (layer F.Cu) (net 9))
 (segment (start 82.55 43.5) (end 82.45 43.4) (width 0.25) (layer F.Cu) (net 9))
 (segment (start 84 43.5) (end 82.55 43.5) (width 0.25) (layer F.Cu) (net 9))
 (segment (start 77.55 106.6) (end 75.1 106.6) (width 0.5) (layer F.Cu) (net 17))
 (segment (start 75.1 106.6) (end 74 105.5) (width 0.5) (layer F.Cu) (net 17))
 (via (at 74 73.5) (size 0.8) (drill 0.4) (layers F.Cu B.Cu) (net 17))
 (segment (start 74 105.5) (end 74 73.5) (width 0.5) (layer F.Cu) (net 17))
 (via (at 74 64.5) (size 0.8) (drill 0.4) (layers F.Cu B.Cu) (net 17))
 (segment (start 74 73.5) (end 74 64.5) (width 0.5) (layer B.Cu) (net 17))
 (segment (start 74 50.15) (end 77.55 46.6) (width 0.5) (layer F.Cu) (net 17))
 (segment (start 74 64.5) (end 74 50.15) (width 0.5) (layer F.Cu) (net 17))
 (segment (start 80 105.85) (end 82.45 103.4) (width 0.5) (layer F.Cu) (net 3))
 (segment (start 80 107.5) (end 80 105.85) (width 0.5) (layer F.Cu) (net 3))
 (segment (start 89.5 117) (end 80 107.5) (width 0.5) (layer F.Cu) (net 3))
 (segment (start 129 117) (end 89.5 117) (width 0.5) (layer F.Cu) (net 3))
 (segment (start 138.4 107.6) (end 129 117) (width 0.5) (layer F.Cu) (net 3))
 (segment (start 138.55 107.6) (end 138.4 107.6) (width 0.5) (layer F.Cu) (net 3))
 (segment (start 142.45 43.4) (end 143.9 43.4) (width 0.5) (layer F.Cu) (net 2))
 (segment (start 143.9 43.4) (end 145.5 45) (width 0.5) (layer F.Cu) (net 2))
 (segment (start 145.5 102.35) (end 143.45 104.4) (width 0.5) (layer F.Cu) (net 2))
 (segment (start 145.5 45) (end 145.5 102.35) (width 0.5) (layer F.Cu) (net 2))
 (via (at 91 70) (size 0.8) (drill 0.4) (layers F.Cu B.Cu) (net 10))
 (segment (start 90.602 70.398) (end 91 70) (width 0.5) (layer F.Cu) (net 10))
 (segment (start 90.602 71.326) (end 90.602 70.398) (width 0.5) (layer F.Cu) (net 10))
 (segment (start 91 70) (end 93 68) (width 0.5) (layer B.Cu) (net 10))
 (via (at 98 66) (size 0.8) (drill 0.4) (layers F.Cu B.Cu) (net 10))
 (segment (start 96 68) (end 98 66) (width 0.5) (layer B.Cu) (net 10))
 (segment (start 93 68) (end 96 68) (width 0.5) (layer B.Cu) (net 10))
 (segment (start 97.160685 64.595) (end 96.202 64.595) (width 0.5) (layer F.Cu) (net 10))
 (segment (start 98 65.434315) (end 97.160685 64.595) (width 0.5) (layer F.Cu) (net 10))
 (segment (start 98 66) (end 98 65.434315) (width 0.5) (layer F.Cu) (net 10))
 (via (at 88 71) (size 0.8) (drill 0.4) (layers F.Cu B.Cu) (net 11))
 (segment (start 89.596 72.596) (end 88 71) (width 0.5) (layer F.Cu) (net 11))
 (segment (start 90.602 72.596) (end 89.596 72.596) (width 0.5) (layer F.Cu) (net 11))
 (segment (start 88 71) (end 93 66) (width 0.5) (layer B.Cu) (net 11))
 (via (at 98 64) (size 0.8) (drill 0.4) (layers F.Cu B.Cu) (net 11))
 (segment (start 96 66) (end 98 64) (width 0.5) (layer B.Cu) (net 11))
 (segment (start 93 66) (end 96 66) (width 0.5) (layer B.Cu) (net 11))
 (segment (start 97.325 63.325) (end 96.202 63.325) (width 0.5) (layer F.Cu) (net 11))
 (segment (start 98 64) (end 97.325 63.325) (width 0.5) (layer F.Cu) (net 11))
 (segment (start 86.686998 62.055) (end 88.902 62.055) (width 0.5) (layer F.Cu) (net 6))
 (segment (start 86.149999 62.591999) (end 86.686998 62.055) (width 0.5) (layer F.Cu) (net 6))
 (segment (start 86.149999 71.113999) (end 86.149999 62.591999) (width 0.5) (layer F.Cu) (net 6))
 (segment (start 88.902 73.866) (end 86.149999 71.113999) (width 0.5) (layer F.Cu) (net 6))
 (segment (start 90.602 73.866) (end 88.902 73.866) (width 0.5) (layer F.Cu) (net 6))
 (via (at 87 63) (size 0.8) (drill 0.4) (layers F.Cu B.Cu) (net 7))
 (segment (start 87.325 63.325) (end 87 63) (width 0.5) (layer F.Cu) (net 7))
 (segment (start 88.902 63.325) (end 87.325 63.325) (width 0.5) (layer F.Cu) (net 7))
 (segment (start 87 63) (end 87 61) (width 0.5) (layer B.Cu) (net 7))
 (segment (start 87 61) (end 89 59) (width 0.5) (layer B.Cu) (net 7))
 (segment (start 89 59) (end 97 59) (width 0.5) (layer B.Cu) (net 7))
 (segment (start 97 59) (end 99 61) (width 0.5) (layer B.Cu) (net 7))
 (segment (start 99 61) (end 104 66) (width 0.5) (layer B.Cu) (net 7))
 (via (at 104 66) (size 0.8) (drill 0.4) (layers F.Cu B.Cu) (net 7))
 (segment (start 107.538 71.4625) (end 106.4625 71.4625) (width 0.5) (layer F.Cu) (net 7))
 (segment (start 104 69) (end 104 66) (width 0.5) (layer F.Cu) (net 7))
 (segment (start 106.4625 71.4625) (end 104 69) (width 0.5) (layer F.Cu) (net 7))
 (segment (start 107.538 71.4625) (end 107.538 80) (width 0.5) (layer F.Cu) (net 7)))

